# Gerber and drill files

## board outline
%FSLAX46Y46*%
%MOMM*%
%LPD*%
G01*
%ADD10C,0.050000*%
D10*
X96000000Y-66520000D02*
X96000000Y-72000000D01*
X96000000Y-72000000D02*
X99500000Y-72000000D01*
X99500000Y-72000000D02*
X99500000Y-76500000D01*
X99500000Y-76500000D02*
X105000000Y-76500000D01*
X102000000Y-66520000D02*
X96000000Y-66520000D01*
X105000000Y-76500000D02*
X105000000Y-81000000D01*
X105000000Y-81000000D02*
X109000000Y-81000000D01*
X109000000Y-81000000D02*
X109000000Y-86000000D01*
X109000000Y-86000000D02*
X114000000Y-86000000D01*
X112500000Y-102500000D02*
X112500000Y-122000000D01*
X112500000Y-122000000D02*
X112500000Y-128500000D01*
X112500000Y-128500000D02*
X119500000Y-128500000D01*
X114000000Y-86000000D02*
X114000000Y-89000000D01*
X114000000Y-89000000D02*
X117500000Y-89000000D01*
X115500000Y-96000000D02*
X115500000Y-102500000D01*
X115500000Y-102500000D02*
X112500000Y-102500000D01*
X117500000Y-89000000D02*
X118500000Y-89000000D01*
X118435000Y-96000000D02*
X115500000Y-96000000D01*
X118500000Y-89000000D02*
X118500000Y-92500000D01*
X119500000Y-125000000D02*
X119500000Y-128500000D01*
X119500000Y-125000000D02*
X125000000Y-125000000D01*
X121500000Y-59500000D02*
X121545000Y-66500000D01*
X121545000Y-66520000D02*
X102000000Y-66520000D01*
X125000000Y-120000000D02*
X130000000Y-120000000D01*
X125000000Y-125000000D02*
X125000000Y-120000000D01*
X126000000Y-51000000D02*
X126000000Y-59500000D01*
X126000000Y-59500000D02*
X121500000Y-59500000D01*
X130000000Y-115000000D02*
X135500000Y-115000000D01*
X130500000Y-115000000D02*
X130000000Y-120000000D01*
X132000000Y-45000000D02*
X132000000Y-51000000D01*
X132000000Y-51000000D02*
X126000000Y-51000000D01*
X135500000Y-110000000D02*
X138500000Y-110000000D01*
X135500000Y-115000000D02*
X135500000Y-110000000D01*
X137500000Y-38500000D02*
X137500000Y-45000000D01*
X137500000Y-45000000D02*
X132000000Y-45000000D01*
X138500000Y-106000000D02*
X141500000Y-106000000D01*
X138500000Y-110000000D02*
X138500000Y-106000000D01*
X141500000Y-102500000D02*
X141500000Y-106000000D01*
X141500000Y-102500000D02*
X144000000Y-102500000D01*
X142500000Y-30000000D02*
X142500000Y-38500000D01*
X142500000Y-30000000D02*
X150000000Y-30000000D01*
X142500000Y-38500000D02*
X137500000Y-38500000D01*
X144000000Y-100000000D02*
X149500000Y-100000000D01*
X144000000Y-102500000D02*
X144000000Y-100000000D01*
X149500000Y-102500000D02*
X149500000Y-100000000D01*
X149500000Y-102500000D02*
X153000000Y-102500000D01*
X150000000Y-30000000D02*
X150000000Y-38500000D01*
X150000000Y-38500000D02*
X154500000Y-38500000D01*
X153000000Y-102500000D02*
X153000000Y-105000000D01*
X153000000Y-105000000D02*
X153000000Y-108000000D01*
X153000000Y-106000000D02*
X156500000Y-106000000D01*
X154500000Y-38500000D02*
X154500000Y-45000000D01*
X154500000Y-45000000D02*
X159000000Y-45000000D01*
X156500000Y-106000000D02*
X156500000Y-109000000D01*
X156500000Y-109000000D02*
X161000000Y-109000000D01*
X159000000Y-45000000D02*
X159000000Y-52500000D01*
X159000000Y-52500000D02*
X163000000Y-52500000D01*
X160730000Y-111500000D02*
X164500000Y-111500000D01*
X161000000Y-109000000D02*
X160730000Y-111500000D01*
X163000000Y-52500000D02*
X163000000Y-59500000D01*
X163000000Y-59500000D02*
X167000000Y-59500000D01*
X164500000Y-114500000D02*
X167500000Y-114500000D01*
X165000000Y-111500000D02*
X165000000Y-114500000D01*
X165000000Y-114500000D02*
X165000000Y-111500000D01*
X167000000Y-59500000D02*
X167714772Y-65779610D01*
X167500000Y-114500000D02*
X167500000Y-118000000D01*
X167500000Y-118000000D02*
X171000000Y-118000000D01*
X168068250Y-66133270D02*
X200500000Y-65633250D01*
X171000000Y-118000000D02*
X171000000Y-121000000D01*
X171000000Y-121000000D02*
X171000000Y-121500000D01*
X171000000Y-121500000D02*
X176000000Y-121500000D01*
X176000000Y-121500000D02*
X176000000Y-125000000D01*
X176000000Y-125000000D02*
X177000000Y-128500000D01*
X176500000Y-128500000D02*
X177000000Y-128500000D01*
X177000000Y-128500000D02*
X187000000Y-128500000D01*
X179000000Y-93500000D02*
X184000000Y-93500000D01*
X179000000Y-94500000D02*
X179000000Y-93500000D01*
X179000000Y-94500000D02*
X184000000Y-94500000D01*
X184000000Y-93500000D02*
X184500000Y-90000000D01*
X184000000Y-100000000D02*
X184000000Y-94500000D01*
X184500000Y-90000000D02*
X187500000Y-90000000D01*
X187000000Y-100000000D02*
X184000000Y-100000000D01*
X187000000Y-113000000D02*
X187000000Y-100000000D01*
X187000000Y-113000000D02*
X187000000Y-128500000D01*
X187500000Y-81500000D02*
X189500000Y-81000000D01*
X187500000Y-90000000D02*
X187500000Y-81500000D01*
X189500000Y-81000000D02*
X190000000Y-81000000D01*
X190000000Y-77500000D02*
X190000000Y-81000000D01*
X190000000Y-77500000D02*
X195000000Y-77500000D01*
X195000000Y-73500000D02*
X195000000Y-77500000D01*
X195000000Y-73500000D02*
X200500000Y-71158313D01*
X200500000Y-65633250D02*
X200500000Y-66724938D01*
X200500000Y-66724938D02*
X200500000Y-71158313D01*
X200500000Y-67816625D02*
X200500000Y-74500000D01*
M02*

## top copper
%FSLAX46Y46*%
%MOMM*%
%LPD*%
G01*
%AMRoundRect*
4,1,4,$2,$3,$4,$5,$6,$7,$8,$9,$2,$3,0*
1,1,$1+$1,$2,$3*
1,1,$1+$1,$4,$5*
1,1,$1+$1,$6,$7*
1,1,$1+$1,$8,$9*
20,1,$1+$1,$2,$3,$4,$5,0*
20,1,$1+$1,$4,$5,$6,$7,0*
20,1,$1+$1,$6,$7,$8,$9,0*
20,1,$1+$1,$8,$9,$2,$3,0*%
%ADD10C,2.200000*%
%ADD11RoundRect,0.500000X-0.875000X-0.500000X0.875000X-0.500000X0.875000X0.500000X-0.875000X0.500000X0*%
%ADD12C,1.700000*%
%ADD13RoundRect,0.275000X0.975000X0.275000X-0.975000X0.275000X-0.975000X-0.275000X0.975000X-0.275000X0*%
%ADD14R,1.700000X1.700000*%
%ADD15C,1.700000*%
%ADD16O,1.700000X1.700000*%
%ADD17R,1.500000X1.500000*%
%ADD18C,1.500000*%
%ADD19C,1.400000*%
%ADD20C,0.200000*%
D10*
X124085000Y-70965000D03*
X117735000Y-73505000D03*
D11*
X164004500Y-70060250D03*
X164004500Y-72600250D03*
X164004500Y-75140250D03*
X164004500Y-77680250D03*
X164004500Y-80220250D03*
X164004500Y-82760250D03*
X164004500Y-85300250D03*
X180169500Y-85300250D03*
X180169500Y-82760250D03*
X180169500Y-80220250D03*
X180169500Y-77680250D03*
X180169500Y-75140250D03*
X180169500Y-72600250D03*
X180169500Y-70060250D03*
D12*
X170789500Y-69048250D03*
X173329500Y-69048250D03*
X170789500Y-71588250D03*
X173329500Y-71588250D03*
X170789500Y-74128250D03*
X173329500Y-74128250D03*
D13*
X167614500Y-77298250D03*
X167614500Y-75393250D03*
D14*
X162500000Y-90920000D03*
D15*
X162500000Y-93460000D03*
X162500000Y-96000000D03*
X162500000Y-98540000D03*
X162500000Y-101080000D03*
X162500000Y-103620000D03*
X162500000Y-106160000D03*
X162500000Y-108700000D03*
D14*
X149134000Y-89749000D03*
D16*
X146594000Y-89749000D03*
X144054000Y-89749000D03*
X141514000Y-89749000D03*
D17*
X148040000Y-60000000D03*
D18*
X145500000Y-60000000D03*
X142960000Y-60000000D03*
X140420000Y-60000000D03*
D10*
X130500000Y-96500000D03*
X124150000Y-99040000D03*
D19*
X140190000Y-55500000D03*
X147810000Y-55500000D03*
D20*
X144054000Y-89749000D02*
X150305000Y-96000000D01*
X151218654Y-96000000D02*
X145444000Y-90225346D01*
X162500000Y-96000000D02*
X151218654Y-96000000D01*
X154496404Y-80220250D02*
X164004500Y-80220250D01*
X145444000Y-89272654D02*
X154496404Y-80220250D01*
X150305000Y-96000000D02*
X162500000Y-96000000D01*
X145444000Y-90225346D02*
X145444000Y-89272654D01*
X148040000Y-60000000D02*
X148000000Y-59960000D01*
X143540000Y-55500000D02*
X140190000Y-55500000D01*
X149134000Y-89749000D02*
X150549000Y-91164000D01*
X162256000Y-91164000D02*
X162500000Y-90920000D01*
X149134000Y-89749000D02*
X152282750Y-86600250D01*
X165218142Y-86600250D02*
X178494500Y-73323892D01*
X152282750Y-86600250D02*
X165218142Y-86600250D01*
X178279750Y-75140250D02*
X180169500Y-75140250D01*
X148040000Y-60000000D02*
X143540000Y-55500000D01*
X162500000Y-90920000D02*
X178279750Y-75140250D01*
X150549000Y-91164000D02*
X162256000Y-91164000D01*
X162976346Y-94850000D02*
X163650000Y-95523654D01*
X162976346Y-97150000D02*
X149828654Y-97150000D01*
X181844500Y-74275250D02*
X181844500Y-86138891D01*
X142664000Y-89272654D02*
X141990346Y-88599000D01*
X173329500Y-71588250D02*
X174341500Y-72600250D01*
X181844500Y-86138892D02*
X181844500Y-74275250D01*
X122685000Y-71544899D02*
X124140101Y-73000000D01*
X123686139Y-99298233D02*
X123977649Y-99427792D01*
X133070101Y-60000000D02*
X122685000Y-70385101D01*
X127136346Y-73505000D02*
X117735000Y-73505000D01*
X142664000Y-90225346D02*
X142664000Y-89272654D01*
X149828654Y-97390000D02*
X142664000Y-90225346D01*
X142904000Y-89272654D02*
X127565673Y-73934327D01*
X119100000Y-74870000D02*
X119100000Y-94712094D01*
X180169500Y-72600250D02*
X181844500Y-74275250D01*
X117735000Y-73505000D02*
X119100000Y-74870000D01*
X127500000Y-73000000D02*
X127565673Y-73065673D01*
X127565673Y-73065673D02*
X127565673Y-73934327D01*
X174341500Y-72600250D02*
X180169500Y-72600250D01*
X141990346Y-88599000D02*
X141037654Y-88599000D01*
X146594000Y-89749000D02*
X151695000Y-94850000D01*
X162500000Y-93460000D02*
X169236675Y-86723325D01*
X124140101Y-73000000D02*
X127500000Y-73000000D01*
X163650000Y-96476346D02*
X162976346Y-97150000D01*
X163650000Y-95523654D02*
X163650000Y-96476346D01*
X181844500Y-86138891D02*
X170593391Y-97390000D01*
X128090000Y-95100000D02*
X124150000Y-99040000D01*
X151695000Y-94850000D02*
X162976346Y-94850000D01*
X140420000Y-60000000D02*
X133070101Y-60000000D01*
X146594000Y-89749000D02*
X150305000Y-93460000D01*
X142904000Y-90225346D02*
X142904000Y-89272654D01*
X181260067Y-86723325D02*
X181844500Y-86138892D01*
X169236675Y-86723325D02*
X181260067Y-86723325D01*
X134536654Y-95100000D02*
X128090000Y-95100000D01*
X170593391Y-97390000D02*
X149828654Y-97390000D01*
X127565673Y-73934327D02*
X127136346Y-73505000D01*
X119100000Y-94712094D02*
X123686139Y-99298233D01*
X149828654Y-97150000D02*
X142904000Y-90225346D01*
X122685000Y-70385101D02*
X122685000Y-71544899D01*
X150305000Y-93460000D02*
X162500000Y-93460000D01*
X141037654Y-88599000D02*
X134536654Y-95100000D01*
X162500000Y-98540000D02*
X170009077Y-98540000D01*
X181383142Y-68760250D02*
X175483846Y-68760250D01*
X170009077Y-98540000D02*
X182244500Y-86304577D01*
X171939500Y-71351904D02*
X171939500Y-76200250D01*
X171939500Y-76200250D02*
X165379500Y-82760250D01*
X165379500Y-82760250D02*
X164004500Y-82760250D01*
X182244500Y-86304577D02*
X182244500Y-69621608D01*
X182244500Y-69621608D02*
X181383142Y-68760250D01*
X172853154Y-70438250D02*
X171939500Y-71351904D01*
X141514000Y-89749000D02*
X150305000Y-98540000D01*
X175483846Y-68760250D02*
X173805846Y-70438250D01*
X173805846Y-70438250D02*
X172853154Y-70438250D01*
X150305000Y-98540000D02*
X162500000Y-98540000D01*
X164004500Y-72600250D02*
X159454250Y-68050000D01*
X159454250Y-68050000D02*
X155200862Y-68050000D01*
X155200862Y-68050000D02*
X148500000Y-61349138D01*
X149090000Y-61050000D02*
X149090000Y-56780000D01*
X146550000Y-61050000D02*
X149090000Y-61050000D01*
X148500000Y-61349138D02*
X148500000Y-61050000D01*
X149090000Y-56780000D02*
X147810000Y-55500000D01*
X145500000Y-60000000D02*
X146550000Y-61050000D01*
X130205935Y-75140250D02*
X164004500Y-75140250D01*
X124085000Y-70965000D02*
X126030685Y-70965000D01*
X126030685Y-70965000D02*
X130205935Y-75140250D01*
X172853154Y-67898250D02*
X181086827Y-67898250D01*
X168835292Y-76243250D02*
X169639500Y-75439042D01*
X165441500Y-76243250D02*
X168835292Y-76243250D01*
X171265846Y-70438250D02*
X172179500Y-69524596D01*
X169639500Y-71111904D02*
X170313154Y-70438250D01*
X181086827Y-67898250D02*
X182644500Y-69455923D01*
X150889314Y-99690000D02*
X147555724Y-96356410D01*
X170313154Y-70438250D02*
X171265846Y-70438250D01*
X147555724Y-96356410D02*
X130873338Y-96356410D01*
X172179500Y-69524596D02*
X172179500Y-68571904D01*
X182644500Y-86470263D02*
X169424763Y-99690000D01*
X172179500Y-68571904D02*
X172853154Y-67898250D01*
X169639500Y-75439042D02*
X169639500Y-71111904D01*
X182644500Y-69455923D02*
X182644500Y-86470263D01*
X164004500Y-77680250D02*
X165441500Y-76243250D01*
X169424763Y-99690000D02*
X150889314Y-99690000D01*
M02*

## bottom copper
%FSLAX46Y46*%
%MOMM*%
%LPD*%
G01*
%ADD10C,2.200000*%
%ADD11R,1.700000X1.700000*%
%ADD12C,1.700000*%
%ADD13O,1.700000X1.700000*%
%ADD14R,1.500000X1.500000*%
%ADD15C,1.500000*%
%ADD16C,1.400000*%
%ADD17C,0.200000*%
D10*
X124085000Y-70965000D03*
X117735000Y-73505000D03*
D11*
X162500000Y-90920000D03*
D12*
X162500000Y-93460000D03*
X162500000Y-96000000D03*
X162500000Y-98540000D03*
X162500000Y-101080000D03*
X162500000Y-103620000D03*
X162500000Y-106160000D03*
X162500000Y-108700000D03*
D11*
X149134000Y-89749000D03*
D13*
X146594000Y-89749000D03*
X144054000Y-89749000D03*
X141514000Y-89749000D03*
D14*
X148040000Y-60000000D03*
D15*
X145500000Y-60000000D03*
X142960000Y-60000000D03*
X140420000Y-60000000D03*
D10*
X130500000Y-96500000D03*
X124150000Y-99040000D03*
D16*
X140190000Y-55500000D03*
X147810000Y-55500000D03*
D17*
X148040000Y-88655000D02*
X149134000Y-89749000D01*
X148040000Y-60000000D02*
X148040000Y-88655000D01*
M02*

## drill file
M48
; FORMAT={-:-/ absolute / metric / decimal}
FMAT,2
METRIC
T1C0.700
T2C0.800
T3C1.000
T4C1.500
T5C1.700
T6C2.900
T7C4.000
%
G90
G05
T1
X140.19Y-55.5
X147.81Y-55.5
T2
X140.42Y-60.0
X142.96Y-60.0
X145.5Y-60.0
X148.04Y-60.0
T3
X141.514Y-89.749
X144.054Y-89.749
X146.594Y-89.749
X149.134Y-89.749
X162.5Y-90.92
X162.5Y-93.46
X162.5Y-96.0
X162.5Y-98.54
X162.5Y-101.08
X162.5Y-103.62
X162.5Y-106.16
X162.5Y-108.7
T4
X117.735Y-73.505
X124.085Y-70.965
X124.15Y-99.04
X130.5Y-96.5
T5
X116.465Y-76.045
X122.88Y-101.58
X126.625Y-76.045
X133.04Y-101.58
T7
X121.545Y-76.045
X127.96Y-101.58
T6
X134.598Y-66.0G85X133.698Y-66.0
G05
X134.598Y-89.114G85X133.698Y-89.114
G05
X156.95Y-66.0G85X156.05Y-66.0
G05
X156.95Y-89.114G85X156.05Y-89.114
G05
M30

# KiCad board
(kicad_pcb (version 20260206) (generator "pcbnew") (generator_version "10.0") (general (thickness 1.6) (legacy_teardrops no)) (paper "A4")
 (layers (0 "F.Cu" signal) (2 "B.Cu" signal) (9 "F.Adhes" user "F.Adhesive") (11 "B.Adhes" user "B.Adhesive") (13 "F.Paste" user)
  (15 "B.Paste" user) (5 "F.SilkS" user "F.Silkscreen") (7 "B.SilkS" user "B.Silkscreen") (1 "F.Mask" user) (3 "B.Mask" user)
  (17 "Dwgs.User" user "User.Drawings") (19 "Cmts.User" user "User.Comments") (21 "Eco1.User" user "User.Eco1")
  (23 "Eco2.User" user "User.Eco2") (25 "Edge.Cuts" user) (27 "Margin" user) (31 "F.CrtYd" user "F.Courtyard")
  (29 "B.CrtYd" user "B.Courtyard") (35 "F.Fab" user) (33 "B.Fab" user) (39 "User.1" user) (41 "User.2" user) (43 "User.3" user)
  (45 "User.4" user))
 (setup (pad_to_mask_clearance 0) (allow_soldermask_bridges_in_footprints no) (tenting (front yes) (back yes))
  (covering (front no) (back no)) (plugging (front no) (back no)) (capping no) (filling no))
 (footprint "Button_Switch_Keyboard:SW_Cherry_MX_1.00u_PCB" (layer "F.Cu") (at 124.085 70.965)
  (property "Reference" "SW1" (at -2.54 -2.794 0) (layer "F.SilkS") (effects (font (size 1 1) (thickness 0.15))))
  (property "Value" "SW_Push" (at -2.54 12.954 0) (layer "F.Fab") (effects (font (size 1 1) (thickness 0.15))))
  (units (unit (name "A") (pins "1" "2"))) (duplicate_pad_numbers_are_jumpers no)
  (pad "" np_thru_hole circle (at -7.62 5.08) (size 1.7 1.7) (drill 1.7) (layers "*.Cu" "*.Mask"))
  (pad "" np_thru_hole circle (at -2.54 5.08) (size 4 4) (drill 4) (layers "*.Cu" "*.Mask"))
  (pad "" np_thru_hole circle (at 2.54 5.08) (size 1.7 1.7) (drill 1.7) (layers "*.Cu" "*.Mask"))
  (pad "1" thru_hole circle (at 0 0) (size 2.2 2.2) (drill 1.5) (layers "*.Cu" "*.Mask") (remove_unused_layers no) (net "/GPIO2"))
  (pad "2" thru_hole circle (at -6.35 2.54) (size 2.2 2.2) (drill 1.5) (layers "*.Cu" "*.Mask") (remove_unused_layers no) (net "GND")))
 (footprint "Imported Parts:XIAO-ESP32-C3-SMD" (layer "F.Cu") (at 163.1695 88.18025)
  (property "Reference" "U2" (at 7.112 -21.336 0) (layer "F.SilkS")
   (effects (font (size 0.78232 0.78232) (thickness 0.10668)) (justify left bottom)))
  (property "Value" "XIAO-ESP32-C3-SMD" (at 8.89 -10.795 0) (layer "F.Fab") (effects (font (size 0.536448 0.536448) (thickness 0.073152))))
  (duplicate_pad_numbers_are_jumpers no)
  (pad "1" smd roundrect (at 0.835 -18.12) (size 2.75 2) (layers "F.Cu" "F.Mask" "F.Paste") (roundrect_rratio 0.25)
   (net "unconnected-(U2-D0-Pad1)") (solder_mask_margin 0.0508) (thermal_bridge_angle 45))
  (pad "2" smd roundrect (at 0.835 -15.58) (size 2.75 2) (layers "F.Cu" "F.Mask" "F.Paste") (roundrect_rratio 0.25) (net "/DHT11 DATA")
   (solder_mask_margin 0.0508) (thermal_bridge_angle 45))
  (pad "3" smd roundrect (at 0.835 -13.04) (size 2.75 2) (layers "F.Cu" "F.Mask" "F.Paste") (roundrect_rratio 0.25) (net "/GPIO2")
   (solder_mask_margin 0.0508) (thermal_bridge_angle 45))
  (pad "4" smd roundrect (at 0.835 -10.5) (size 2.75 2) (layers "F.Cu" "F.Mask" "F.Paste") (roundrect_rratio 0.25) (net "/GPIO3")
   (solder_mask_margin 0.0508) (thermal_bridge_angle 45))
  (pad "5" smd roundrect (at 0.835 -7.96) (size 2.75 2) (layers "F.Cu" "F.Mask" "F.Paste") (roundrect_rratio 0.25) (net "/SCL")
   (solder_mask_margin 0.0508) (thermal_bridge_angle 45))
  (pad "6" smd roundrect (at 0.835 -5.42) (size 2.75 2) (layers "F.Cu" "F.Mask" "F.Paste") (roundrect_rratio 0.25) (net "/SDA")
   (solder_mask_margin 0.0508) (thermal_bridge_angle 45))
  (pad "7" smd roundrect (at 0.835 -2.88) (size 2.75 2) (layers "F.Cu" "F.Mask" "F.Paste") (roundrect_rratio 0.25)
   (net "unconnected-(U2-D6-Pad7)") (solder_mask_margin 0.0508) (thermal_bridge_angle 45))
  (pad "8" smd roundrect (at 17 -2.88) (size 2.75 2) (layers "F.Cu" "F.Mask" "F.Paste") (roundrect_rratio 0.25)
   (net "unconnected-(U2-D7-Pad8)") (solder_mask_margin 0.0508) (thermal_bridge_angle 45))
  (pad "9" smd roundrect (at 17 -5.42) (size 2.75 2) (layers "F.Cu" "F.Mask" "F.Paste") (roundrect_rratio 0.25)
   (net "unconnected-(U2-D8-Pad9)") (solder_mask_margin 0.0508) (thermal_bridge_angle 45))
  (pad "10" smd roundrect (at 17 -7.96) (size 2.75 2) (layers "F.Cu" "F.Mask" "F.Paste") (roundrect_rratio 0.25)
   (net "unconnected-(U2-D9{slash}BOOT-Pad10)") (solder_mask_margin 0.0508) (thermal_bridge_angle 45))
  (pad "11" smd roundrect (at 17 -10.5) (size 2.75 2) (layers "F.Cu" "F.Mask" "F.Paste") (roundrect_rratio 0.25)
   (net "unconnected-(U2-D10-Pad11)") (solder_mask_margin 0.0508) (thermal_bridge_angle 45))
  (pad "12" smd roundrect (at 17 -13.04) (size 2.75 2) (layers "F.Cu" "F.Mask" "F.Paste") (roundrect_rratio 0.25) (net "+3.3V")
   (solder_mask_margin 0.0508) (thermal_bridge_angle 45))
  (pad "13" smd roundrect (at 17 -15.58) (size 2.75 2) (layers "F.Cu" "F.Mask" "F.Paste") (roundrect_rratio 0.25) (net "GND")
   (solder_mask_margin 0.0508) (thermal_bridge_angle 45))
  (pad "14" smd roundrect (at 17 -18.12) (size 2.75 2) (layers "F.Cu" "F.Mask" "F.Paste") (roundrect_rratio 0.25) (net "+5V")
   (solder_mask_margin 0.0508) (thermal_bridge_angle 45))
  (pad "15" smd circle (at 7.62 -19.132) (size 1.7 1.7) (layers "F.Cu" "F.Mask" "F.Paste") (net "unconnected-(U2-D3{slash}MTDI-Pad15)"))
  (pad "16" smd circle (at 10.16 -19.132) (size 1.7 1.7) (layers "F.Cu" "F.Mask" "F.Paste") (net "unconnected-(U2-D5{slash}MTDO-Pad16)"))
  (pad "17" smd circle (at 7.62 -16.592) (size 1.7 1.7) (layers "F.Cu" "F.Mask" "F.Paste") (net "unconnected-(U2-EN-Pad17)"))
  (pad "18" smd circle (at 10.16 -16.592) (size 1.7 1.7) (layers "F.Cu" "F.Mask" "F.Paste") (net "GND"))
  (pad "19" smd circle (at 7.62 -14.052) (size 1.7 1.7) (layers "F.Cu" "F.Mask" "F.Paste") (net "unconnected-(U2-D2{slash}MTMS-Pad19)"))
  (pad "20" smd circle (at 10.16 -14.052) (size 1.7 1.7) (layers "F.Cu" "F.Mask" "F.Paste") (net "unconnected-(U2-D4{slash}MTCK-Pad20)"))
  (pad "21" smd roundrect (at 4.445 -10.882 180) (size 2.5 1.1) (layers "F.Cu" "F.Mask" "F.Paste") (roundrect_rratio 0.25)
   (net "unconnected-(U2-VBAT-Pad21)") (thermal_bridge_angle 45))
  (pad "22" smd roundrect (at 4.445 -12.787 180) (size 2.5 1.1) (layers "F.Cu" "F.Mask" "F.Paste") (roundrect_rratio 0.25)
   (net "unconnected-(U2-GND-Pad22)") (thermal_bridge_angle 45)))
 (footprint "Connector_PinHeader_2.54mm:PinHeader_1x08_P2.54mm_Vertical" (layer "F.Cu") (at 162.5 90.92)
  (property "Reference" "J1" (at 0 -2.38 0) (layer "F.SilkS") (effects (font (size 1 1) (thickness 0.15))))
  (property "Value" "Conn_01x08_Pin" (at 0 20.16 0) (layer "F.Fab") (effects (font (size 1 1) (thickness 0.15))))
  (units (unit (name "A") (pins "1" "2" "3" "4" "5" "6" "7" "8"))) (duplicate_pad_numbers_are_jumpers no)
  (pad "1" thru_hole rect (at 0 0) (size 1.7 1.7) (drill 1) (layers "*.Cu" "*.Mask") (remove_unused_layers no) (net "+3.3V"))
  (pad "2" thru_hole circle (at 0 2.54) (size 1.7 1.7) (drill 1) (layers "*.Cu" "*.Mask") (remove_unused_layers no) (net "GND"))
  (pad "3" thru_hole circle (at 0 5.08) (size 1.7 1.7) (drill 1) (layers "*.Cu" "*.Mask") (remove_unused_layers no) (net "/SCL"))
  (pad "4" thru_hole circle (at 0 7.62) (size 1.7 1.7) (drill 1) (layers "*.Cu" "*.Mask") (remove_unused_layers no) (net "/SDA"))
  (pad "5" thru_hole circle (at 0 10.16) (size 1.7 1.7) (drill 1) (layers "*.Cu" "*.Mask") (remove_unused_layers no)
   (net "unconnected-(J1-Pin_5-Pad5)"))
  (pad "6" thru_hole circle (at 0 12.7) (size 1.7 1.7) (drill 1) (layers "*.Cu" "*.Mask") (remove_unused_layers no)
   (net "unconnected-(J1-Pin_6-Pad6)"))
  (pad "7" thru_hole circle (at 0 15.24) (size 1.7 1.7) (drill 1) (layers "*.Cu" "*.Mask") (remove_unused_layers no)
   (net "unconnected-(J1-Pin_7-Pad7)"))
  (pad "8" thru_hole circle (at 0 17.78) (size 1.7 1.7) (drill 1) (layers "*.Cu" "*.Mask") (remove_unused_layers no)
   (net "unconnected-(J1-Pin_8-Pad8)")))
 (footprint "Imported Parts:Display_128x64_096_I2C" (layer "F.Cu") (at 145.324 89.749 180)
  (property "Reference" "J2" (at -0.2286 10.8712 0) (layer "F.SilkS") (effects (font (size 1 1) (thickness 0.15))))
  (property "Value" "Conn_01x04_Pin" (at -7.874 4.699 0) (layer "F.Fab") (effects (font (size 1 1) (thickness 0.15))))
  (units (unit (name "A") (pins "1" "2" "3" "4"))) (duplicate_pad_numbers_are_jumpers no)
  (pad "" np_thru_hole oval (at -11.176 0.635 180) (size 3.8 2.9) (drill oval 3.8 2.9) (layers "*.Cu" "*.Mask"))
  (pad "" np_thru_hole oval (at -11.176 23.749 180) (size 3.8 2.9) (drill oval 3.8 2.9) (layers "*.Cu" "*.Mask"))
  (pad "" np_thru_hole oval (at 11.176 0.635 180) (size 3.8 2.9) (drill oval 3.8 2.9) (layers "*.Cu" "*.Mask"))
  (pad "" np_thru_hole oval (at 11.176 23.749 180) (size 3.8 2.9) (drill oval 3.8 2.9) (layers "*.Cu" "*.Mask"))
  (pad "1" thru_hole rect (at -3.81 0 270) (size 1.7 1.7) (drill 1) (layers "*.Cu" "*.Mask") (remove_unused_layers no) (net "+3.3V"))
  (pad "2" thru_hole oval (at -1.27 0 270) (size 1.7 1.7) (drill 1) (layers "*.Cu" "*.Mask") (remove_unused_layers no) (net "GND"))
  (pad "3" thru_hole oval (at 1.27 0 270) (size 1.7 1.7) (drill 1) (layers "*.Cu" "*.Mask") (remove_unused_layers no) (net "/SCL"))
  (pad "4" thru_hole oval (at 3.81 0 270) (size 1.7 1.7) (drill 1) (layers "*.Cu" "*.Mask") (remove_unused_layers no) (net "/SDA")))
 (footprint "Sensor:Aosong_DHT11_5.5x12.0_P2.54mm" (layer "F.Cu") (at 148.04 60 -90)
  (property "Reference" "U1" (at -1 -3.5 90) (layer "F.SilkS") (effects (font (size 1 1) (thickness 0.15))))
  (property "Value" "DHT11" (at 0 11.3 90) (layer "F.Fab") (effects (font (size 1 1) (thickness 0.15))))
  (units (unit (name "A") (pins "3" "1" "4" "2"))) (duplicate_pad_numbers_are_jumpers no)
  (pad "1" thru_hole rect (at 0 0 270) (size 1.5 1.5) (drill 0.8) (layers "*.Cu" "*.Mask") (remove_unused_layers no) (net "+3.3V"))
  (pad "2" thru_hole circle (at 0 2.54 270) (size 1.5 1.5) (drill 0.8) (layers "*.Cu" "*.Mask") (remove_unused_layers no)
   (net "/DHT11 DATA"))
  (pad "3" thru_hole circle (at 0 5.08 270) (size 1.5 1.5) (drill 0.8) (layers "*.Cu" "*.Mask") (remove_unused_layers no)
   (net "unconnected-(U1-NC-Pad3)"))
  (pad "4" thru_hole circle (at 0 7.62 270) (size 1.5 1.5) (drill 0.8) (layers "*.Cu" "*.Mask") (remove_unused_layers no) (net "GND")))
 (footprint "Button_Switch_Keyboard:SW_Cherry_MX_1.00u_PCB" (layer "F.Cu") (at 130.5 96.5)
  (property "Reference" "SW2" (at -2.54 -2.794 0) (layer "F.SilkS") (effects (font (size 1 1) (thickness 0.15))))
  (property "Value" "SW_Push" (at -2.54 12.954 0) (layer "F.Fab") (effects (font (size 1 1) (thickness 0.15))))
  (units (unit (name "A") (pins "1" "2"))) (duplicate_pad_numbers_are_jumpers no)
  (pad "" np_thru_hole circle (at -7.62 5.08) (size 1.7 1.7) (drill 1.7) (layers "*.Cu" "*.Mask"))
  (pad "" np_thru_hole circle (at -2.54 5.08) (size 4 4) (drill 4) (layers "*.Cu" "*.Mask"))
  (pad "" np_thru_hole circle (at 2.54 5.08) (size 1.7 1.7) (drill 1.7) (layers "*.Cu" "*.Mask"))
  (pad "1" thru_hole circle (at 0 0) (size 2.2 2.2) (drill 1.5) (layers "*.Cu" "*.Mask") (remove_unused_layers no) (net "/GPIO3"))
  (pad "2" thru_hole circle (at -6.35 2.54) (size 2.2 2.2) (drill 1.5) (layers "*.Cu" "*.Mask") (remove_unused_layers no) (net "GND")))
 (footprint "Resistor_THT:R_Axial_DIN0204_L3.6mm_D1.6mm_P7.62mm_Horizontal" (layer "F.Cu") (at 140.19 55.5)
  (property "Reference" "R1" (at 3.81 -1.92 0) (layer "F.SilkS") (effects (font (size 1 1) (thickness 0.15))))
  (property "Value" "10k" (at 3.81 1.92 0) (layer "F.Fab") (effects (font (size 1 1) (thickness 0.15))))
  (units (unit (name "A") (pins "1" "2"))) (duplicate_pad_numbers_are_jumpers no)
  (pad "1" thru_hole circle (at 0 0) (size 1.4 1.4) (drill 0.7) (layers "*.Cu" "*.Mask") (remove_unused_layers no) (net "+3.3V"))
  (pad "2" thru_hole circle (at 7.62 0) (size 1.4 1.4) (drill 0.7) (layers "*.Cu" "*.Mask") (remove_unused_layers no) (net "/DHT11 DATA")))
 (gr_line (start 96 66.52) (end 96 72) (stroke (width 0.05) (type default)) (layer "Edge.Cuts"))
 (gr_line (start 96 72) (end 99.5 72) (stroke (width 0.05) (type default)) (layer "Edge.Cuts"))
 (gr_line (start 99.5 72) (end 99.5 76.5) (stroke (width 0.05) (type default)) (layer "Edge.Cuts"))
 (gr_line (start 99.5 76.5) (end 105 76.5) (stroke (width 0.05) (type default)) (layer "Edge.Cuts"))
 (gr_line (start 102 66.52) (end 96 66.52) (stroke (width 0.05) (type default)) (layer "Edge.Cuts"))
 (gr_line (start 105 76.5) (end 105 81) (stroke (width 0.05) (type default)) (layer "Edge.Cuts"))
 (gr_line (start 105 81) (end 109 81) (stroke (width 0.05) (type default)) (layer "Edge.Cuts"))
 (gr_line (start 109 81) (end 109 86) (stroke (width 0.05) (type default)) (layer "Edge.Cuts"))
 (gr_line (start 109 86) (end 114 86) (stroke (width 0.05) (type default)) (layer "Edge.Cuts"))
 (gr_line (start 112.5 102.5) (end 112.5 122) (stroke (width 0.05) (type default)) (layer "Edge.Cuts"))
 (gr_line (start 112.5 122) (end 112.5 128.5) (stroke (width 0.05) (type default)) (layer "Edge.Cuts"))
 (gr_line (start 112.5 128.5) (end 119.5 128.5) (stroke (width 0.05) (type default)) (layer "Edge.Cuts"))
 (gr_line (start 114 86) (end 114 89) (stroke (width 0.05) (type default)) (layer "Edge.Cuts"))
 (gr_line (start 114 89) (end 117.5 89) (stroke (width 0.05) (type default)) (layer "Edge.Cuts"))
 (gr_line (start 115.5 96) (end 115.5 102.5) (stroke (width 0.05) (type default)) (layer "Edge.Cuts"))
 (gr_line (start 115.5 102.5) (end 112.5 102.5) (stroke (width 0.05) (type default)) (layer "Edge.Cuts"))
 (gr_line (start 117.5 89) (end 118.5 89) (stroke (width 0.05) (type default)) (layer "Edge.Cuts"))
 (gr_line (start 118.435 96) (end 115.5 96) (stroke (width 0.05) (type default)) (layer "Edge.Cuts"))
 (gr_line (start 118.5 89) (end 118.5 92.5) (stroke (width 0.05) (type default)) (layer "Edge.Cuts"))
 (gr_line (start 119.5 125) (end 119.5 128.5) (stroke (width 0.05) (type default)) (layer "Edge.Cuts"))
 (gr_line (start 119.5 125) (end 125 125) (stroke (width 0.05) (type default)) (layer "Edge.Cuts"))
 (gr_line (start 121.5 59.5) (end 121.545 66.5) (stroke (width 0.05) (type default)) (layer "Edge.Cuts"))
 (gr_line (start 121.545 66.52) (end 102 66.52) (stroke (width 0.05) (type default)) (layer "Edge.Cuts"))
 (gr_line (start 125 120) (end 130 120) (stroke (width 0.05) (type default)) (layer "Edge.Cuts"))
 (gr_line (start 125 125) (end 125 120) (stroke (width 0.05) (type default)) (layer "Edge.Cuts"))
 (gr_line (start 126 51) (end 126 59.5) (stroke (width 0.05) (type default)) (layer "Edge.Cuts"))
 (gr_line (start 126 59.5) (end 121.5 59.5) (stroke (width 0.05) (type default)) (layer "Edge.Cuts"))
 (gr_line (start 130 115) (end 135.5 115) (stroke (width 0.05) (type default)) (layer "Edge.Cuts"))
 (gr_line (start 130.5 115) (end 130 120) (stroke (width 0.05) (type default)) (layer "Edge.Cuts"))
 (gr_line (start 132 45) (end 132 51) (stroke (width 0.05) (type default)) (layer "Edge.Cuts"))
 (gr_line (start 132 51) (end 126 51) (stroke (width 0.05) (type default)) (layer "Edge.Cuts"))
 (gr_line (start 135.5 110) (end 138.5 110) (stroke (width 0.05) (type default)) (layer "Edge.Cuts"))
 (gr_line (start 135.5 115) (end 135.5 110) (stroke (width 0.05) (type default)) (layer "Edge.Cuts"))
 (gr_line (start 137.5 38.5) (end 137.5 45) (stroke (width 0.05) (type default)) (layer "Edge.Cuts"))
 (gr_line (start 137.5 45) (end 132 45) (stroke (width 0.05) (type default)) (layer "Edge.Cuts"))
 (gr_line (start 138.5 106) (end 141.5 106) (stroke (width 0.05) (type default)) (layer "Edge.Cuts"))
 (gr_line (start 138.5 110) (end 138.5 106) (stroke (width 0.05) (type default)) (layer "Edge.Cuts"))
 (gr_line (start 141.5 102.5) (end 141.5 106) (stroke (width 0.05) (type default)) (layer "Edge.Cuts"))
 (gr_line (start 141.5 102.5) (end 144 102.5) (stroke (width 0.05) (type default)) (layer "Edge.Cuts"))
 (gr_line (start 142.5 30) (end 142.5 38.5) (stroke (width 0.05) (type default)) (layer "Edge.Cuts"))
 (gr_line (start 142.5 30) (end 150 30) (stroke (width 0.05) (type default)) (layer "Edge.Cuts"))
 (gr_line (start 142.5 38.5) (end 137.5 38.5) (stroke (width 0.05) (type default)) (layer "Edge.Cuts"))
 (gr_line (start 144 100) (end 149.5 100) (stroke (width 0.05) (type default)) (layer "Edge.Cuts"))
 (gr_line (start 144 102.5) (end 144 100) (stroke (width 0.05) (type default)) (layer "Edge.Cuts"))
 (gr_line (start 149.5 102.5) (end 149.5 100) (stroke (width 0.05) (type default)) (layer "Edge.Cuts"))
 (gr_line (start 149.5 102.5) (end 153 102.5) (stroke (width 0.05) (type default)) (layer "Edge.Cuts"))
 (gr_line (start 150 30) (end 150 38.5) (stroke (width 0.05) (type default)) (layer "Edge.Cuts"))
 (gr_line (start 150 38.5) (end 154.5 38.5) (stroke (width 0.05) (type default)) (layer "Edge.Cuts"))
 (gr_line (start 153 102.5) (end 153 105) (stroke (width 0.05) (type default)) (layer "Edge.Cuts"))
 (gr_line (start 153 105) (end 153 108) (stroke (width 0.05) (type default)) (layer "Edge.Cuts"))
 (gr_line (start 153 106) (end 156.5 106) (stroke (width 0.05) (type default)) (layer "Edge.Cuts"))
 (gr_line (start 154.5 38.5) (end 154.5 45) (stroke (width 0.05) (type default)) (layer "Edge.Cuts"))
 (gr_line (start 154.5 45) (end 159 45) (stroke (width 0.05) (type default)) (layer "Edge.Cuts"))
 (gr_line (start 156.5 106) (end 156.5 109) (stroke (width 0.05) (type default)) (layer "Edge.Cuts"))
 (gr_line (start 156.5 109) (end 161 109) (stroke (width 0.05) (type default)) (layer "Edge.Cuts"))
 (gr_line (start 159 45) (end 159 52.5) (stroke (width 0.05) (type default)) (layer "Edge.Cuts"))
 (gr_line (start 159 52.5) (end 163 52.5) (stroke (width 0.05) (type default)) (layer "Edge.Cuts"))
 (gr_line (start 160.73 111.5) (end 164.5 111.5) (stroke (width 0.05) (type default)) (layer "Edge.Cuts"))
 (gr_line (start 161 109) (end 160.73 111.5) (stroke (width 0.05) (type default)) (layer "Edge.Cuts"))
 (gr_line (start 163 52.5) (end 163 59.5) (stroke (width 0.05) (type default)) (layer "Edge.Cuts"))
 (gr_line (start 163 59.5) (end 167 59.5) (stroke (width 0.05) (type default)) (layer "Edge.Cuts"))
 (gr_line (start 164.5 114.5) (end 167.5 114.5) (stroke (width 0.05) (type default)) (layer "Edge.Cuts"))
 (gr_line (start 165 111.5) (end 165 114.5) (stroke (width 0.05) (type default)) (layer "Edge.Cuts"))
 (gr_line (start 165 114.5) (end 165 111.5) (stroke (width 0.05) (type default)) (layer "Edge.Cuts"))
 (gr_line (start 167 59.5) (end 167.714772 65.77961) (stroke (width 0.05) (type default)) (layer "Edge.Cuts"))
 (gr_line (start 167.5 114.5) (end 167.5 118) (stroke (width 0.05) (type default)) (layer "Edge.Cuts"))
 (gr_line (start 167.5 118) (end 171 118) (stroke (width 0.05) (type default)) (layer "Edge.Cuts"))
 (gr_line (start 168.06825 66.13327) (end 200.5 65.63325) (stroke (width 0.05) (type default)) (layer "Edge.Cuts"))
 (gr_line (start 171 118) (end 171 121) (stroke (width 0.05) (type default)) (layer "Edge.Cuts"))
 (gr_line (start 171 121) (end 171 121.5) (stroke (width 0.05) (type default)) (layer "Edge.Cuts"))
 (gr_line (start 171 121.5) (end 176 121.5) (stroke (width 0.05) (type default)) (layer "Edge.Cuts"))
 (gr_line (start 176 121.5) (end 176 125) (stroke (width 0.05) (type default)) (layer "Edge.Cuts"))
 (gr_line (start 176 125) (end 177 128.5) (stroke (width 0.05) (type default)) (layer "Edge.Cuts"))
 (gr_line (start 176.5 128.5) (end 177 128.5) (stroke (width 0.05) (type default)) (layer "Edge.Cuts"))
 (gr_line (start 177 128.5) (end 187 128.5) (stroke (width 0.05) (type default)) (layer "Edge.Cuts"))
 (gr_line (start 179 93.5) (end 184 93.5) (stroke (width 0.05) (type default)) (layer "Edge.Cuts"))
 (gr_line (start 179 94.5) (end 179 93.5) (stroke (width 0.05) (type default)) (layer "Edge.Cuts"))
 (gr_line (start 179 94.5) (end 184 94.5) (stroke (width 0.05) (type default)) (layer "Edge.Cuts"))
 (gr_line (start 184 93.5) (end 184.5 90) (stroke (width 0.05) (type default)) (layer "Edge.Cuts"))
 (gr_line (start 184 100) (end 184 94.5) (stroke (width 0.05) (type default)) (layer "Edge.Cuts"))
 (gr_line (start 184.5 90) (end 187.5 90) (stroke (width 0.05) (type default)) (layer "Edge.Cuts"))
 (gr_line (start 187 100) (end 184 100) (stroke (width 0.05) (type default)) (layer "Edge.Cuts"))
 (gr_line (start 187 113) (end 187 100) (stroke (width 0.05) (type default)) (layer "Edge.Cuts"))
 (gr_line (start 187 113) (end 187 128.5) (stroke (width 0.05) (type default)) (layer "Edge.Cuts"))
 (gr_line (start 187.5 81.5) (end 189.5 81) (stroke (width 0.05) (type default)) (layer "Edge.Cuts"))
 (gr_line (start 187.5 90) (end 187.5 81.5) (stroke (width 0.05) (type default)) (layer "Edge.Cuts"))
 (gr_line (start 189.5 81) (end 190 81) (stroke (width 0.05) (type default)) (layer "Edge.Cuts"))
 (gr_line (start 190 77.5) (end 190 81) (stroke (width 0.05) (type default)) (layer "Edge.Cuts"))
 (gr_line (start 190 77.5) (end 195 77.5) (stroke (width 0.05) (type default)) (layer "Edge.Cuts"))
 (gr_line (start 195 73.5) (end 195 77.5) (stroke (width 0.05) (type default)) (layer "Edge.Cuts"))
 (gr_line (start 195 73.5) (end 200.5 71.158313) (stroke (width 0.05) (type default)) (layer "Edge.Cuts"))
 (gr_line (start 200.5 65.63325) (end 200.5 66.724938) (stroke (width 0.05) (type default)) (layer "Edge.Cuts"))
 (gr_line (start 200.5 66.724938) (end 200.5 71.158313) (stroke (width 0.05) (type default)) (layer "Edge.Cuts"))
 (gr_line (start 200.5 67.816625) (end 200.5 74.5) (stroke (width 0.05) (type default)) (layer "Edge.Cuts"))
 (segment (start 144.054 89.749) (end 150.305 96) (width 0.2) (layer "F.Cu") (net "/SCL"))
 (segment (start 151.218654 96) (end 145.444 90.225346) (width 0.2) (layer "F.Cu") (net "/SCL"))
 (segment (start 162.5 96) (end 151.218654 96) (width 0.2) (layer "F.Cu") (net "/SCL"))
 (segment (start 154.496404 80.22025) (end 164.0045 80.22025) (width 0.2) (layer "F.Cu") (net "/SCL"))
 (segment (start 145.444 89.272654) (end 154.496404 80.22025) (width 0.2) (layer "F.Cu") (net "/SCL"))
 (segment (start 150.305 96) (end 162.5 96) (width 0.2) (layer "F.Cu") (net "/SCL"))
 (segment (start 145.444 90.225346) (end 145.444 89.272654) (width 0.2) (layer "F.Cu") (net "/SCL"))
 (segment (start 148.04 60) (end 148 59.96) (width 0.2) (layer "F.Cu") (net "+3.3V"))
 (segment (start 143.54 55.5) (end 140.19 55.5) (width 0.2) (layer "F.Cu") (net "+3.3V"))
 (segment (start 149.134 89.749) (end 150.549 91.164) (width 0.2) (layer "F.Cu") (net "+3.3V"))
 (segment (start 162.256 91.164) (end 162.5 90.92) (width 0.2) (layer "F.Cu") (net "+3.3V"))
 (segment (start 149.134 89.749) (end 152.28275 86.60025) (width 0.2) (layer "F.Cu") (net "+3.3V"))
 (segment (start 165.218142 86.60025) (end 178.4945 73.323892) (width 0.2) (layer "F.Cu") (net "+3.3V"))
 (segment (start 152.28275 86.60025) (end 165.218142 86.60025) (width 0.2) (layer "F.Cu") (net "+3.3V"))
 (segment (start 178.27975 75.14025) (end 180.1695 75.14025) (width 0.2) (layer "F.Cu") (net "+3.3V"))
 (segment (start 148.04 60) (end 143.54 55.5) (width 0.2) (layer "F.Cu") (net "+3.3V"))
 (segment (start 162.5 90.92) (end 178.27975 75.14025) (width 0.2) (layer "F.Cu") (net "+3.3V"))
 (segment (start 150.549 91.164) (end 162.256 91.164) (width 0.2) (layer "F.Cu") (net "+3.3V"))
 (segment (start 148.04 88.655) (end 149.134 89.749) (width 0.2) (layer "B.Cu") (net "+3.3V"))
 (segment (start 148.04 60) (end 148.04 88.655) (width 0.2) (layer "B.Cu") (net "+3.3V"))
 (segment (start 162.976346 94.85) (end 163.65 95.523654) (width 0.2) (layer "F.Cu") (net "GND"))
 (segment (start 162.976346 97.15) (end 149.828654 97.15) (width 0.2) (layer "F.Cu") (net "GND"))
 (segment (start 181.8445 74.27525) (end 181.8445 86.138891) (width 0.2) (layer "F.Cu") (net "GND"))
 (segment (start 142.664 89.272654) (end 141.990346 88.599) (width 0.2) (layer "F.Cu") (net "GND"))
 (segment (start 173.3295 71.58825) (end 174.3415 72.60025) (width 0.2) (layer "F.Cu") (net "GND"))
 (segment (start 181.8445 86.138892) (end 181.8445 74.27525) (width 0.2) (layer "F.Cu") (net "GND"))
 (segment (start 122.685 71.544899) (end 124.140101 73) (width 0.2) (layer "F.Cu") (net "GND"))
 (segment (start 123.686139 99.298233) (end 123.977649 99.427792) (width 0.2) (layer "F.Cu") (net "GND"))
 (segment (start 133.070101 60) (end 122.685 70.385101) (width 0.2) (layer "F.Cu") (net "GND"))
 (segment (start 127.136346 73.505) (end 117.735 73.505) (width 0.2) (layer "F.Cu") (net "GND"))
 (segment (start 142.664 90.225346) (end 142.664 89.272654) (width 0.2) (layer "F.Cu") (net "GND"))
 (segment (start 149.828654 97.39) (end 142.664 90.225346) (width 0.2) (layer "F.Cu") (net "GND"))
 (segment (start 142.904 89.272654) (end 127.565673 73.934327) (width 0.2) (layer "F.Cu") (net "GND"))
 (segment (start 119.1 74.87) (end 119.1 94.712094) (width 0.2) (layer "F.Cu") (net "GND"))
 (segment (start 180.1695 72.60025) (end 181.8445 74.27525) (width 0.2) (layer "F.Cu") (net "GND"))
 (segment (start 117.735 73.505) (end 119.1 74.87) (width 0.2) (layer "F.Cu") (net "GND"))
 (segment (start 127.5 73) (end 127.565673 73.065673) (width 0.2) (layer "F.Cu") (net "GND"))
 (segment (start 127.565673 73.065673) (end 127.565673 73.934327) (width 0.2) (layer "F.Cu") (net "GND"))
 (segment (start 174.3415 72.60025) (end 180.1695 72.60025) (width 0.2) (layer "F.Cu") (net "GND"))
 (segment (start 141.990346 88.599) (end 141.037654 88.599) (width 0.2) (layer "F.Cu") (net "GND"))
 (segment (start 146.594 89.749) (end 151.695 94.85) (width 0.2) (layer "F.Cu") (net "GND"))
 (segment (start 162.5 93.46) (end 169.236675 86.723325) (width 0.2) (layer "F.Cu") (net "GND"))
 (segment (start 124.140101 73) (end 127.5 73) (width 0.2) (layer "F.Cu") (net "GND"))
 (segment (start 163.65 96.476346) (end 162.976346 97.15) (width 0.2) (layer "F.Cu") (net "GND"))
 (segment (start 163.65 95.523654) (end 163.65 96.476346) (width 0.2) (layer "F.Cu") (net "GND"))
 (segment (start 181.8445 86.138891) (end 170.593391 97.39) (width 0.2) (layer "F.Cu") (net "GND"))
 (segment (start 128.09 95.1) (end 124.15 99.04) (width 0.2) (layer "F.Cu") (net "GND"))
 (segment (start 151.695 94.85) (end 162.976346 94.85) (width 0.2) (layer "F.Cu") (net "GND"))
 (segment (start 140.42 60) (end 133.070101 60) (width 0.2) (layer "F.Cu") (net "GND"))
 (segment (start 146.594 89.749) (end 150.305 93.46) (width 0.2) (layer "F.Cu") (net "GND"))
 (segment (start 142.904 90.225346) (end 142.904 89.272654) (width 0.2) (layer "F.Cu") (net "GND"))
 (segment (start 181.260067 86.723325) (end 181.8445 86.138892) (width 0.2) (layer "F.Cu") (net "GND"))
 (segment (start 169.236675 86.723325) (end 181.260067 86.723325) (width 0.2) (layer "F.Cu") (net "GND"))
 (segment (start 134.536654 95.1) (end 128.09 95.1) (width 0.2) (layer "F.Cu") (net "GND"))
 (segment (start 170.593391 97.39) (end 149.828654 97.39) (width 0.2) (layer "F.Cu") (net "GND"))
 (segment (start 127.565673 73.934327) (end 127.136346 73.505) (width 0.2) (layer "F.Cu") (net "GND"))
 (segment (start 119.1 94.712094) (end 123.686139 99.298233) (width 0.2) (layer "F.Cu") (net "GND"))
 (segment (start 149.828654 97.15) (end 142.904 90.225346) (width 0.2) (layer "F.Cu") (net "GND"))
 (segment (start 122.685 70.385101) (end 122.685 71.544899) (width 0.2) (layer "F.Cu") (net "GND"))
 (segment (start 150.305 93.46) (end 162.5 93.46) (width 0.2) (layer "F.Cu") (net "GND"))
 (segment (start 141.037654 88.599) (end 134.536654 95.1) (width 0.2) (layer "F.Cu") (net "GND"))
 (segment (start 162.5 98.54) (end 170.009077 98.54) (width 0.2) (layer "F.Cu") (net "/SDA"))
 (segment (start 181.383142 68.76025) (end 175.483846 68.76025) (width 0.2) (layer "F.Cu") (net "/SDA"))
 (segment (start 170.009077 98.54) (end 182.2445 86.304577) (width 0.2) (layer "F.Cu") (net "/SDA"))
 (segment (start 171.9395 71.351904) (end 171.9395 76.20025) (width 0.2) (layer "F.Cu") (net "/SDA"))
 (segment (start 171.9395 76.20025) (end 165.3795 82.76025) (width 0.2) (layer "F.Cu") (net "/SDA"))
 (segment (start 165.3795 82.76025) (end 164.0045 82.76025) (width 0.2) (layer "F.Cu") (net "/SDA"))
 (segment (start 182.2445 86.304577) (end 182.2445 69.621608) (width 0.2) (layer "F.Cu") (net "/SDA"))
 (segment (start 182.2445 69.621608) (end 181.383142 68.76025) (width 0.2) (layer "F.Cu") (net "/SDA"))
 (segment (start 172.853154 70.43825) (end 171.9395 71.351904) (width 0.2) (layer "F.Cu") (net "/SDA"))
 (segment (start 141.514 89.749) (end 150.305 98.54) (width 0.2) (layer "F.Cu") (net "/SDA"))
 (segment (start 175.483846 68.76025) (end 173.805846 70.43825) (width 0.2) (layer "F.Cu") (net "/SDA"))
 (segment (start 173.805846 70.43825) (end 172.853154 70.43825) (width 0.2) (layer "F.Cu") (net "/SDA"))
 (segment (start 150.305 98.54) (end 162.5 98.54) (width 0.2) (layer "F.Cu") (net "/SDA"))
 (segment (start 164.0045 72.60025) (end 159.45425 68.05) (width 0.2) (layer "F.Cu") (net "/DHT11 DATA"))
 (segment (start 159.45425 68.05) (end 155.200862 68.05) (width 0.2) (layer "F.Cu") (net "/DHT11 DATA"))
 (segment (start 155.200862 68.05) (end 148.5 61.349138) (width 0.2) (layer "F.Cu") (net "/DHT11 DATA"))
 (segment (start 149.09 61.05) (end 149.09 56.78) (width 0.2) (layer "F.Cu") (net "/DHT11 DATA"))
 (segment (start 146.55 61.05) (end 149.09 61.05) (width 0.2) (layer "F.Cu") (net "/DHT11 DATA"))
 (segment (start 148.5 61.349138) (end 148.5 61.05) (width 0.2) (layer "F.Cu") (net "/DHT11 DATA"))
 (segment (start 149.09 56.78) (end 147.81 55.5) (width 0.2) (layer "F.Cu") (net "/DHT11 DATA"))
 (segment (start 145.5 60) (end 146.55 61.05) (width 0.2) (layer "F.Cu") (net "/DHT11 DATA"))
 (segment (start 130.205935 75.14025) (end 164.0045 75.14025) (width 0.2) (layer "F.Cu") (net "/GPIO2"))
 (segment (start 124.085 70.965) (end 126.030685 70.965) (width 0.2) (layer "F.Cu") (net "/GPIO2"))
 (segment (start 126.030685 70.965) (end 130.205935 75.14025) (width 0.2) (layer "F.Cu") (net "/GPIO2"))
 (segment (start 172.853154 67.89825) (end 181.086827 67.89825) (width 0.2) (layer "F.Cu") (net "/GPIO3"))
 (segment (start 168.835292 76.24325) (end 169.6395 75.439042) (width 0.2) (layer "F.Cu") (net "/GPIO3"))
 (segment (start 165.4415 76.24325) (end 168.835292 76.24325) (width 0.2) (layer "F.Cu") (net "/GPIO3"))
 (segment (start 171.265846 70.43825) (end 172.1795 69.524596) (width 0.2) (layer "F.Cu") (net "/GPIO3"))
 (segment (start 169.6395 71.111904) (end 170.313154 70.43825) (width 0.2) (layer "F.Cu") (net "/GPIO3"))
 (segment (start 181.086827 67.89825) (end 182.6445 69.455923) (width 0.2) (layer "F.Cu") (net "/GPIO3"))
 (segment (start 150.889314 99.69) (end 147.555724 96.35641) (width 0.2) (layer "F.Cu") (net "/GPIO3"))
 (segment (start 170.313154 70.43825) (end 171.265846 70.43825) (width 0.2) (layer "F.Cu") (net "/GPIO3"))
 (segment (start 147.555724 96.35641) (end 130.873338 96.35641) (width 0.2) (layer "F.Cu") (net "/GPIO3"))
 (segment (start 172.1795 69.524596) (end 172.1795 68.571904) (width 0.2) (layer "F.Cu") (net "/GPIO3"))
 (segment (start 182.6445 86.470263) (end 169.424763 99.69) (width 0.2) (layer "F.Cu") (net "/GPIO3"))
 (segment (start 172.1795 68.571904) (end 172.853154 67.89825) (width 0.2) (layer "F.Cu") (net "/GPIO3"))
 (segment (start 169.6395 75.439042) (end 169.6395 71.111904) (width 0.2) (layer "F.Cu") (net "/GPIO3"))
 (segment (start 182.6445 69.455923) (end 182.6445 86.470263) (width 0.2) (layer "F.Cu") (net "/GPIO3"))
 (segment (start 164.0045 77.68025) (end 165.4415 76.24325) (width 0.2) (layer "F.Cu") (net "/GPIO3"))
 (segment (start 169.424763 99.69) (end 150.889314 99.69) (width 0.2) (layer "F.Cu") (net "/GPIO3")))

